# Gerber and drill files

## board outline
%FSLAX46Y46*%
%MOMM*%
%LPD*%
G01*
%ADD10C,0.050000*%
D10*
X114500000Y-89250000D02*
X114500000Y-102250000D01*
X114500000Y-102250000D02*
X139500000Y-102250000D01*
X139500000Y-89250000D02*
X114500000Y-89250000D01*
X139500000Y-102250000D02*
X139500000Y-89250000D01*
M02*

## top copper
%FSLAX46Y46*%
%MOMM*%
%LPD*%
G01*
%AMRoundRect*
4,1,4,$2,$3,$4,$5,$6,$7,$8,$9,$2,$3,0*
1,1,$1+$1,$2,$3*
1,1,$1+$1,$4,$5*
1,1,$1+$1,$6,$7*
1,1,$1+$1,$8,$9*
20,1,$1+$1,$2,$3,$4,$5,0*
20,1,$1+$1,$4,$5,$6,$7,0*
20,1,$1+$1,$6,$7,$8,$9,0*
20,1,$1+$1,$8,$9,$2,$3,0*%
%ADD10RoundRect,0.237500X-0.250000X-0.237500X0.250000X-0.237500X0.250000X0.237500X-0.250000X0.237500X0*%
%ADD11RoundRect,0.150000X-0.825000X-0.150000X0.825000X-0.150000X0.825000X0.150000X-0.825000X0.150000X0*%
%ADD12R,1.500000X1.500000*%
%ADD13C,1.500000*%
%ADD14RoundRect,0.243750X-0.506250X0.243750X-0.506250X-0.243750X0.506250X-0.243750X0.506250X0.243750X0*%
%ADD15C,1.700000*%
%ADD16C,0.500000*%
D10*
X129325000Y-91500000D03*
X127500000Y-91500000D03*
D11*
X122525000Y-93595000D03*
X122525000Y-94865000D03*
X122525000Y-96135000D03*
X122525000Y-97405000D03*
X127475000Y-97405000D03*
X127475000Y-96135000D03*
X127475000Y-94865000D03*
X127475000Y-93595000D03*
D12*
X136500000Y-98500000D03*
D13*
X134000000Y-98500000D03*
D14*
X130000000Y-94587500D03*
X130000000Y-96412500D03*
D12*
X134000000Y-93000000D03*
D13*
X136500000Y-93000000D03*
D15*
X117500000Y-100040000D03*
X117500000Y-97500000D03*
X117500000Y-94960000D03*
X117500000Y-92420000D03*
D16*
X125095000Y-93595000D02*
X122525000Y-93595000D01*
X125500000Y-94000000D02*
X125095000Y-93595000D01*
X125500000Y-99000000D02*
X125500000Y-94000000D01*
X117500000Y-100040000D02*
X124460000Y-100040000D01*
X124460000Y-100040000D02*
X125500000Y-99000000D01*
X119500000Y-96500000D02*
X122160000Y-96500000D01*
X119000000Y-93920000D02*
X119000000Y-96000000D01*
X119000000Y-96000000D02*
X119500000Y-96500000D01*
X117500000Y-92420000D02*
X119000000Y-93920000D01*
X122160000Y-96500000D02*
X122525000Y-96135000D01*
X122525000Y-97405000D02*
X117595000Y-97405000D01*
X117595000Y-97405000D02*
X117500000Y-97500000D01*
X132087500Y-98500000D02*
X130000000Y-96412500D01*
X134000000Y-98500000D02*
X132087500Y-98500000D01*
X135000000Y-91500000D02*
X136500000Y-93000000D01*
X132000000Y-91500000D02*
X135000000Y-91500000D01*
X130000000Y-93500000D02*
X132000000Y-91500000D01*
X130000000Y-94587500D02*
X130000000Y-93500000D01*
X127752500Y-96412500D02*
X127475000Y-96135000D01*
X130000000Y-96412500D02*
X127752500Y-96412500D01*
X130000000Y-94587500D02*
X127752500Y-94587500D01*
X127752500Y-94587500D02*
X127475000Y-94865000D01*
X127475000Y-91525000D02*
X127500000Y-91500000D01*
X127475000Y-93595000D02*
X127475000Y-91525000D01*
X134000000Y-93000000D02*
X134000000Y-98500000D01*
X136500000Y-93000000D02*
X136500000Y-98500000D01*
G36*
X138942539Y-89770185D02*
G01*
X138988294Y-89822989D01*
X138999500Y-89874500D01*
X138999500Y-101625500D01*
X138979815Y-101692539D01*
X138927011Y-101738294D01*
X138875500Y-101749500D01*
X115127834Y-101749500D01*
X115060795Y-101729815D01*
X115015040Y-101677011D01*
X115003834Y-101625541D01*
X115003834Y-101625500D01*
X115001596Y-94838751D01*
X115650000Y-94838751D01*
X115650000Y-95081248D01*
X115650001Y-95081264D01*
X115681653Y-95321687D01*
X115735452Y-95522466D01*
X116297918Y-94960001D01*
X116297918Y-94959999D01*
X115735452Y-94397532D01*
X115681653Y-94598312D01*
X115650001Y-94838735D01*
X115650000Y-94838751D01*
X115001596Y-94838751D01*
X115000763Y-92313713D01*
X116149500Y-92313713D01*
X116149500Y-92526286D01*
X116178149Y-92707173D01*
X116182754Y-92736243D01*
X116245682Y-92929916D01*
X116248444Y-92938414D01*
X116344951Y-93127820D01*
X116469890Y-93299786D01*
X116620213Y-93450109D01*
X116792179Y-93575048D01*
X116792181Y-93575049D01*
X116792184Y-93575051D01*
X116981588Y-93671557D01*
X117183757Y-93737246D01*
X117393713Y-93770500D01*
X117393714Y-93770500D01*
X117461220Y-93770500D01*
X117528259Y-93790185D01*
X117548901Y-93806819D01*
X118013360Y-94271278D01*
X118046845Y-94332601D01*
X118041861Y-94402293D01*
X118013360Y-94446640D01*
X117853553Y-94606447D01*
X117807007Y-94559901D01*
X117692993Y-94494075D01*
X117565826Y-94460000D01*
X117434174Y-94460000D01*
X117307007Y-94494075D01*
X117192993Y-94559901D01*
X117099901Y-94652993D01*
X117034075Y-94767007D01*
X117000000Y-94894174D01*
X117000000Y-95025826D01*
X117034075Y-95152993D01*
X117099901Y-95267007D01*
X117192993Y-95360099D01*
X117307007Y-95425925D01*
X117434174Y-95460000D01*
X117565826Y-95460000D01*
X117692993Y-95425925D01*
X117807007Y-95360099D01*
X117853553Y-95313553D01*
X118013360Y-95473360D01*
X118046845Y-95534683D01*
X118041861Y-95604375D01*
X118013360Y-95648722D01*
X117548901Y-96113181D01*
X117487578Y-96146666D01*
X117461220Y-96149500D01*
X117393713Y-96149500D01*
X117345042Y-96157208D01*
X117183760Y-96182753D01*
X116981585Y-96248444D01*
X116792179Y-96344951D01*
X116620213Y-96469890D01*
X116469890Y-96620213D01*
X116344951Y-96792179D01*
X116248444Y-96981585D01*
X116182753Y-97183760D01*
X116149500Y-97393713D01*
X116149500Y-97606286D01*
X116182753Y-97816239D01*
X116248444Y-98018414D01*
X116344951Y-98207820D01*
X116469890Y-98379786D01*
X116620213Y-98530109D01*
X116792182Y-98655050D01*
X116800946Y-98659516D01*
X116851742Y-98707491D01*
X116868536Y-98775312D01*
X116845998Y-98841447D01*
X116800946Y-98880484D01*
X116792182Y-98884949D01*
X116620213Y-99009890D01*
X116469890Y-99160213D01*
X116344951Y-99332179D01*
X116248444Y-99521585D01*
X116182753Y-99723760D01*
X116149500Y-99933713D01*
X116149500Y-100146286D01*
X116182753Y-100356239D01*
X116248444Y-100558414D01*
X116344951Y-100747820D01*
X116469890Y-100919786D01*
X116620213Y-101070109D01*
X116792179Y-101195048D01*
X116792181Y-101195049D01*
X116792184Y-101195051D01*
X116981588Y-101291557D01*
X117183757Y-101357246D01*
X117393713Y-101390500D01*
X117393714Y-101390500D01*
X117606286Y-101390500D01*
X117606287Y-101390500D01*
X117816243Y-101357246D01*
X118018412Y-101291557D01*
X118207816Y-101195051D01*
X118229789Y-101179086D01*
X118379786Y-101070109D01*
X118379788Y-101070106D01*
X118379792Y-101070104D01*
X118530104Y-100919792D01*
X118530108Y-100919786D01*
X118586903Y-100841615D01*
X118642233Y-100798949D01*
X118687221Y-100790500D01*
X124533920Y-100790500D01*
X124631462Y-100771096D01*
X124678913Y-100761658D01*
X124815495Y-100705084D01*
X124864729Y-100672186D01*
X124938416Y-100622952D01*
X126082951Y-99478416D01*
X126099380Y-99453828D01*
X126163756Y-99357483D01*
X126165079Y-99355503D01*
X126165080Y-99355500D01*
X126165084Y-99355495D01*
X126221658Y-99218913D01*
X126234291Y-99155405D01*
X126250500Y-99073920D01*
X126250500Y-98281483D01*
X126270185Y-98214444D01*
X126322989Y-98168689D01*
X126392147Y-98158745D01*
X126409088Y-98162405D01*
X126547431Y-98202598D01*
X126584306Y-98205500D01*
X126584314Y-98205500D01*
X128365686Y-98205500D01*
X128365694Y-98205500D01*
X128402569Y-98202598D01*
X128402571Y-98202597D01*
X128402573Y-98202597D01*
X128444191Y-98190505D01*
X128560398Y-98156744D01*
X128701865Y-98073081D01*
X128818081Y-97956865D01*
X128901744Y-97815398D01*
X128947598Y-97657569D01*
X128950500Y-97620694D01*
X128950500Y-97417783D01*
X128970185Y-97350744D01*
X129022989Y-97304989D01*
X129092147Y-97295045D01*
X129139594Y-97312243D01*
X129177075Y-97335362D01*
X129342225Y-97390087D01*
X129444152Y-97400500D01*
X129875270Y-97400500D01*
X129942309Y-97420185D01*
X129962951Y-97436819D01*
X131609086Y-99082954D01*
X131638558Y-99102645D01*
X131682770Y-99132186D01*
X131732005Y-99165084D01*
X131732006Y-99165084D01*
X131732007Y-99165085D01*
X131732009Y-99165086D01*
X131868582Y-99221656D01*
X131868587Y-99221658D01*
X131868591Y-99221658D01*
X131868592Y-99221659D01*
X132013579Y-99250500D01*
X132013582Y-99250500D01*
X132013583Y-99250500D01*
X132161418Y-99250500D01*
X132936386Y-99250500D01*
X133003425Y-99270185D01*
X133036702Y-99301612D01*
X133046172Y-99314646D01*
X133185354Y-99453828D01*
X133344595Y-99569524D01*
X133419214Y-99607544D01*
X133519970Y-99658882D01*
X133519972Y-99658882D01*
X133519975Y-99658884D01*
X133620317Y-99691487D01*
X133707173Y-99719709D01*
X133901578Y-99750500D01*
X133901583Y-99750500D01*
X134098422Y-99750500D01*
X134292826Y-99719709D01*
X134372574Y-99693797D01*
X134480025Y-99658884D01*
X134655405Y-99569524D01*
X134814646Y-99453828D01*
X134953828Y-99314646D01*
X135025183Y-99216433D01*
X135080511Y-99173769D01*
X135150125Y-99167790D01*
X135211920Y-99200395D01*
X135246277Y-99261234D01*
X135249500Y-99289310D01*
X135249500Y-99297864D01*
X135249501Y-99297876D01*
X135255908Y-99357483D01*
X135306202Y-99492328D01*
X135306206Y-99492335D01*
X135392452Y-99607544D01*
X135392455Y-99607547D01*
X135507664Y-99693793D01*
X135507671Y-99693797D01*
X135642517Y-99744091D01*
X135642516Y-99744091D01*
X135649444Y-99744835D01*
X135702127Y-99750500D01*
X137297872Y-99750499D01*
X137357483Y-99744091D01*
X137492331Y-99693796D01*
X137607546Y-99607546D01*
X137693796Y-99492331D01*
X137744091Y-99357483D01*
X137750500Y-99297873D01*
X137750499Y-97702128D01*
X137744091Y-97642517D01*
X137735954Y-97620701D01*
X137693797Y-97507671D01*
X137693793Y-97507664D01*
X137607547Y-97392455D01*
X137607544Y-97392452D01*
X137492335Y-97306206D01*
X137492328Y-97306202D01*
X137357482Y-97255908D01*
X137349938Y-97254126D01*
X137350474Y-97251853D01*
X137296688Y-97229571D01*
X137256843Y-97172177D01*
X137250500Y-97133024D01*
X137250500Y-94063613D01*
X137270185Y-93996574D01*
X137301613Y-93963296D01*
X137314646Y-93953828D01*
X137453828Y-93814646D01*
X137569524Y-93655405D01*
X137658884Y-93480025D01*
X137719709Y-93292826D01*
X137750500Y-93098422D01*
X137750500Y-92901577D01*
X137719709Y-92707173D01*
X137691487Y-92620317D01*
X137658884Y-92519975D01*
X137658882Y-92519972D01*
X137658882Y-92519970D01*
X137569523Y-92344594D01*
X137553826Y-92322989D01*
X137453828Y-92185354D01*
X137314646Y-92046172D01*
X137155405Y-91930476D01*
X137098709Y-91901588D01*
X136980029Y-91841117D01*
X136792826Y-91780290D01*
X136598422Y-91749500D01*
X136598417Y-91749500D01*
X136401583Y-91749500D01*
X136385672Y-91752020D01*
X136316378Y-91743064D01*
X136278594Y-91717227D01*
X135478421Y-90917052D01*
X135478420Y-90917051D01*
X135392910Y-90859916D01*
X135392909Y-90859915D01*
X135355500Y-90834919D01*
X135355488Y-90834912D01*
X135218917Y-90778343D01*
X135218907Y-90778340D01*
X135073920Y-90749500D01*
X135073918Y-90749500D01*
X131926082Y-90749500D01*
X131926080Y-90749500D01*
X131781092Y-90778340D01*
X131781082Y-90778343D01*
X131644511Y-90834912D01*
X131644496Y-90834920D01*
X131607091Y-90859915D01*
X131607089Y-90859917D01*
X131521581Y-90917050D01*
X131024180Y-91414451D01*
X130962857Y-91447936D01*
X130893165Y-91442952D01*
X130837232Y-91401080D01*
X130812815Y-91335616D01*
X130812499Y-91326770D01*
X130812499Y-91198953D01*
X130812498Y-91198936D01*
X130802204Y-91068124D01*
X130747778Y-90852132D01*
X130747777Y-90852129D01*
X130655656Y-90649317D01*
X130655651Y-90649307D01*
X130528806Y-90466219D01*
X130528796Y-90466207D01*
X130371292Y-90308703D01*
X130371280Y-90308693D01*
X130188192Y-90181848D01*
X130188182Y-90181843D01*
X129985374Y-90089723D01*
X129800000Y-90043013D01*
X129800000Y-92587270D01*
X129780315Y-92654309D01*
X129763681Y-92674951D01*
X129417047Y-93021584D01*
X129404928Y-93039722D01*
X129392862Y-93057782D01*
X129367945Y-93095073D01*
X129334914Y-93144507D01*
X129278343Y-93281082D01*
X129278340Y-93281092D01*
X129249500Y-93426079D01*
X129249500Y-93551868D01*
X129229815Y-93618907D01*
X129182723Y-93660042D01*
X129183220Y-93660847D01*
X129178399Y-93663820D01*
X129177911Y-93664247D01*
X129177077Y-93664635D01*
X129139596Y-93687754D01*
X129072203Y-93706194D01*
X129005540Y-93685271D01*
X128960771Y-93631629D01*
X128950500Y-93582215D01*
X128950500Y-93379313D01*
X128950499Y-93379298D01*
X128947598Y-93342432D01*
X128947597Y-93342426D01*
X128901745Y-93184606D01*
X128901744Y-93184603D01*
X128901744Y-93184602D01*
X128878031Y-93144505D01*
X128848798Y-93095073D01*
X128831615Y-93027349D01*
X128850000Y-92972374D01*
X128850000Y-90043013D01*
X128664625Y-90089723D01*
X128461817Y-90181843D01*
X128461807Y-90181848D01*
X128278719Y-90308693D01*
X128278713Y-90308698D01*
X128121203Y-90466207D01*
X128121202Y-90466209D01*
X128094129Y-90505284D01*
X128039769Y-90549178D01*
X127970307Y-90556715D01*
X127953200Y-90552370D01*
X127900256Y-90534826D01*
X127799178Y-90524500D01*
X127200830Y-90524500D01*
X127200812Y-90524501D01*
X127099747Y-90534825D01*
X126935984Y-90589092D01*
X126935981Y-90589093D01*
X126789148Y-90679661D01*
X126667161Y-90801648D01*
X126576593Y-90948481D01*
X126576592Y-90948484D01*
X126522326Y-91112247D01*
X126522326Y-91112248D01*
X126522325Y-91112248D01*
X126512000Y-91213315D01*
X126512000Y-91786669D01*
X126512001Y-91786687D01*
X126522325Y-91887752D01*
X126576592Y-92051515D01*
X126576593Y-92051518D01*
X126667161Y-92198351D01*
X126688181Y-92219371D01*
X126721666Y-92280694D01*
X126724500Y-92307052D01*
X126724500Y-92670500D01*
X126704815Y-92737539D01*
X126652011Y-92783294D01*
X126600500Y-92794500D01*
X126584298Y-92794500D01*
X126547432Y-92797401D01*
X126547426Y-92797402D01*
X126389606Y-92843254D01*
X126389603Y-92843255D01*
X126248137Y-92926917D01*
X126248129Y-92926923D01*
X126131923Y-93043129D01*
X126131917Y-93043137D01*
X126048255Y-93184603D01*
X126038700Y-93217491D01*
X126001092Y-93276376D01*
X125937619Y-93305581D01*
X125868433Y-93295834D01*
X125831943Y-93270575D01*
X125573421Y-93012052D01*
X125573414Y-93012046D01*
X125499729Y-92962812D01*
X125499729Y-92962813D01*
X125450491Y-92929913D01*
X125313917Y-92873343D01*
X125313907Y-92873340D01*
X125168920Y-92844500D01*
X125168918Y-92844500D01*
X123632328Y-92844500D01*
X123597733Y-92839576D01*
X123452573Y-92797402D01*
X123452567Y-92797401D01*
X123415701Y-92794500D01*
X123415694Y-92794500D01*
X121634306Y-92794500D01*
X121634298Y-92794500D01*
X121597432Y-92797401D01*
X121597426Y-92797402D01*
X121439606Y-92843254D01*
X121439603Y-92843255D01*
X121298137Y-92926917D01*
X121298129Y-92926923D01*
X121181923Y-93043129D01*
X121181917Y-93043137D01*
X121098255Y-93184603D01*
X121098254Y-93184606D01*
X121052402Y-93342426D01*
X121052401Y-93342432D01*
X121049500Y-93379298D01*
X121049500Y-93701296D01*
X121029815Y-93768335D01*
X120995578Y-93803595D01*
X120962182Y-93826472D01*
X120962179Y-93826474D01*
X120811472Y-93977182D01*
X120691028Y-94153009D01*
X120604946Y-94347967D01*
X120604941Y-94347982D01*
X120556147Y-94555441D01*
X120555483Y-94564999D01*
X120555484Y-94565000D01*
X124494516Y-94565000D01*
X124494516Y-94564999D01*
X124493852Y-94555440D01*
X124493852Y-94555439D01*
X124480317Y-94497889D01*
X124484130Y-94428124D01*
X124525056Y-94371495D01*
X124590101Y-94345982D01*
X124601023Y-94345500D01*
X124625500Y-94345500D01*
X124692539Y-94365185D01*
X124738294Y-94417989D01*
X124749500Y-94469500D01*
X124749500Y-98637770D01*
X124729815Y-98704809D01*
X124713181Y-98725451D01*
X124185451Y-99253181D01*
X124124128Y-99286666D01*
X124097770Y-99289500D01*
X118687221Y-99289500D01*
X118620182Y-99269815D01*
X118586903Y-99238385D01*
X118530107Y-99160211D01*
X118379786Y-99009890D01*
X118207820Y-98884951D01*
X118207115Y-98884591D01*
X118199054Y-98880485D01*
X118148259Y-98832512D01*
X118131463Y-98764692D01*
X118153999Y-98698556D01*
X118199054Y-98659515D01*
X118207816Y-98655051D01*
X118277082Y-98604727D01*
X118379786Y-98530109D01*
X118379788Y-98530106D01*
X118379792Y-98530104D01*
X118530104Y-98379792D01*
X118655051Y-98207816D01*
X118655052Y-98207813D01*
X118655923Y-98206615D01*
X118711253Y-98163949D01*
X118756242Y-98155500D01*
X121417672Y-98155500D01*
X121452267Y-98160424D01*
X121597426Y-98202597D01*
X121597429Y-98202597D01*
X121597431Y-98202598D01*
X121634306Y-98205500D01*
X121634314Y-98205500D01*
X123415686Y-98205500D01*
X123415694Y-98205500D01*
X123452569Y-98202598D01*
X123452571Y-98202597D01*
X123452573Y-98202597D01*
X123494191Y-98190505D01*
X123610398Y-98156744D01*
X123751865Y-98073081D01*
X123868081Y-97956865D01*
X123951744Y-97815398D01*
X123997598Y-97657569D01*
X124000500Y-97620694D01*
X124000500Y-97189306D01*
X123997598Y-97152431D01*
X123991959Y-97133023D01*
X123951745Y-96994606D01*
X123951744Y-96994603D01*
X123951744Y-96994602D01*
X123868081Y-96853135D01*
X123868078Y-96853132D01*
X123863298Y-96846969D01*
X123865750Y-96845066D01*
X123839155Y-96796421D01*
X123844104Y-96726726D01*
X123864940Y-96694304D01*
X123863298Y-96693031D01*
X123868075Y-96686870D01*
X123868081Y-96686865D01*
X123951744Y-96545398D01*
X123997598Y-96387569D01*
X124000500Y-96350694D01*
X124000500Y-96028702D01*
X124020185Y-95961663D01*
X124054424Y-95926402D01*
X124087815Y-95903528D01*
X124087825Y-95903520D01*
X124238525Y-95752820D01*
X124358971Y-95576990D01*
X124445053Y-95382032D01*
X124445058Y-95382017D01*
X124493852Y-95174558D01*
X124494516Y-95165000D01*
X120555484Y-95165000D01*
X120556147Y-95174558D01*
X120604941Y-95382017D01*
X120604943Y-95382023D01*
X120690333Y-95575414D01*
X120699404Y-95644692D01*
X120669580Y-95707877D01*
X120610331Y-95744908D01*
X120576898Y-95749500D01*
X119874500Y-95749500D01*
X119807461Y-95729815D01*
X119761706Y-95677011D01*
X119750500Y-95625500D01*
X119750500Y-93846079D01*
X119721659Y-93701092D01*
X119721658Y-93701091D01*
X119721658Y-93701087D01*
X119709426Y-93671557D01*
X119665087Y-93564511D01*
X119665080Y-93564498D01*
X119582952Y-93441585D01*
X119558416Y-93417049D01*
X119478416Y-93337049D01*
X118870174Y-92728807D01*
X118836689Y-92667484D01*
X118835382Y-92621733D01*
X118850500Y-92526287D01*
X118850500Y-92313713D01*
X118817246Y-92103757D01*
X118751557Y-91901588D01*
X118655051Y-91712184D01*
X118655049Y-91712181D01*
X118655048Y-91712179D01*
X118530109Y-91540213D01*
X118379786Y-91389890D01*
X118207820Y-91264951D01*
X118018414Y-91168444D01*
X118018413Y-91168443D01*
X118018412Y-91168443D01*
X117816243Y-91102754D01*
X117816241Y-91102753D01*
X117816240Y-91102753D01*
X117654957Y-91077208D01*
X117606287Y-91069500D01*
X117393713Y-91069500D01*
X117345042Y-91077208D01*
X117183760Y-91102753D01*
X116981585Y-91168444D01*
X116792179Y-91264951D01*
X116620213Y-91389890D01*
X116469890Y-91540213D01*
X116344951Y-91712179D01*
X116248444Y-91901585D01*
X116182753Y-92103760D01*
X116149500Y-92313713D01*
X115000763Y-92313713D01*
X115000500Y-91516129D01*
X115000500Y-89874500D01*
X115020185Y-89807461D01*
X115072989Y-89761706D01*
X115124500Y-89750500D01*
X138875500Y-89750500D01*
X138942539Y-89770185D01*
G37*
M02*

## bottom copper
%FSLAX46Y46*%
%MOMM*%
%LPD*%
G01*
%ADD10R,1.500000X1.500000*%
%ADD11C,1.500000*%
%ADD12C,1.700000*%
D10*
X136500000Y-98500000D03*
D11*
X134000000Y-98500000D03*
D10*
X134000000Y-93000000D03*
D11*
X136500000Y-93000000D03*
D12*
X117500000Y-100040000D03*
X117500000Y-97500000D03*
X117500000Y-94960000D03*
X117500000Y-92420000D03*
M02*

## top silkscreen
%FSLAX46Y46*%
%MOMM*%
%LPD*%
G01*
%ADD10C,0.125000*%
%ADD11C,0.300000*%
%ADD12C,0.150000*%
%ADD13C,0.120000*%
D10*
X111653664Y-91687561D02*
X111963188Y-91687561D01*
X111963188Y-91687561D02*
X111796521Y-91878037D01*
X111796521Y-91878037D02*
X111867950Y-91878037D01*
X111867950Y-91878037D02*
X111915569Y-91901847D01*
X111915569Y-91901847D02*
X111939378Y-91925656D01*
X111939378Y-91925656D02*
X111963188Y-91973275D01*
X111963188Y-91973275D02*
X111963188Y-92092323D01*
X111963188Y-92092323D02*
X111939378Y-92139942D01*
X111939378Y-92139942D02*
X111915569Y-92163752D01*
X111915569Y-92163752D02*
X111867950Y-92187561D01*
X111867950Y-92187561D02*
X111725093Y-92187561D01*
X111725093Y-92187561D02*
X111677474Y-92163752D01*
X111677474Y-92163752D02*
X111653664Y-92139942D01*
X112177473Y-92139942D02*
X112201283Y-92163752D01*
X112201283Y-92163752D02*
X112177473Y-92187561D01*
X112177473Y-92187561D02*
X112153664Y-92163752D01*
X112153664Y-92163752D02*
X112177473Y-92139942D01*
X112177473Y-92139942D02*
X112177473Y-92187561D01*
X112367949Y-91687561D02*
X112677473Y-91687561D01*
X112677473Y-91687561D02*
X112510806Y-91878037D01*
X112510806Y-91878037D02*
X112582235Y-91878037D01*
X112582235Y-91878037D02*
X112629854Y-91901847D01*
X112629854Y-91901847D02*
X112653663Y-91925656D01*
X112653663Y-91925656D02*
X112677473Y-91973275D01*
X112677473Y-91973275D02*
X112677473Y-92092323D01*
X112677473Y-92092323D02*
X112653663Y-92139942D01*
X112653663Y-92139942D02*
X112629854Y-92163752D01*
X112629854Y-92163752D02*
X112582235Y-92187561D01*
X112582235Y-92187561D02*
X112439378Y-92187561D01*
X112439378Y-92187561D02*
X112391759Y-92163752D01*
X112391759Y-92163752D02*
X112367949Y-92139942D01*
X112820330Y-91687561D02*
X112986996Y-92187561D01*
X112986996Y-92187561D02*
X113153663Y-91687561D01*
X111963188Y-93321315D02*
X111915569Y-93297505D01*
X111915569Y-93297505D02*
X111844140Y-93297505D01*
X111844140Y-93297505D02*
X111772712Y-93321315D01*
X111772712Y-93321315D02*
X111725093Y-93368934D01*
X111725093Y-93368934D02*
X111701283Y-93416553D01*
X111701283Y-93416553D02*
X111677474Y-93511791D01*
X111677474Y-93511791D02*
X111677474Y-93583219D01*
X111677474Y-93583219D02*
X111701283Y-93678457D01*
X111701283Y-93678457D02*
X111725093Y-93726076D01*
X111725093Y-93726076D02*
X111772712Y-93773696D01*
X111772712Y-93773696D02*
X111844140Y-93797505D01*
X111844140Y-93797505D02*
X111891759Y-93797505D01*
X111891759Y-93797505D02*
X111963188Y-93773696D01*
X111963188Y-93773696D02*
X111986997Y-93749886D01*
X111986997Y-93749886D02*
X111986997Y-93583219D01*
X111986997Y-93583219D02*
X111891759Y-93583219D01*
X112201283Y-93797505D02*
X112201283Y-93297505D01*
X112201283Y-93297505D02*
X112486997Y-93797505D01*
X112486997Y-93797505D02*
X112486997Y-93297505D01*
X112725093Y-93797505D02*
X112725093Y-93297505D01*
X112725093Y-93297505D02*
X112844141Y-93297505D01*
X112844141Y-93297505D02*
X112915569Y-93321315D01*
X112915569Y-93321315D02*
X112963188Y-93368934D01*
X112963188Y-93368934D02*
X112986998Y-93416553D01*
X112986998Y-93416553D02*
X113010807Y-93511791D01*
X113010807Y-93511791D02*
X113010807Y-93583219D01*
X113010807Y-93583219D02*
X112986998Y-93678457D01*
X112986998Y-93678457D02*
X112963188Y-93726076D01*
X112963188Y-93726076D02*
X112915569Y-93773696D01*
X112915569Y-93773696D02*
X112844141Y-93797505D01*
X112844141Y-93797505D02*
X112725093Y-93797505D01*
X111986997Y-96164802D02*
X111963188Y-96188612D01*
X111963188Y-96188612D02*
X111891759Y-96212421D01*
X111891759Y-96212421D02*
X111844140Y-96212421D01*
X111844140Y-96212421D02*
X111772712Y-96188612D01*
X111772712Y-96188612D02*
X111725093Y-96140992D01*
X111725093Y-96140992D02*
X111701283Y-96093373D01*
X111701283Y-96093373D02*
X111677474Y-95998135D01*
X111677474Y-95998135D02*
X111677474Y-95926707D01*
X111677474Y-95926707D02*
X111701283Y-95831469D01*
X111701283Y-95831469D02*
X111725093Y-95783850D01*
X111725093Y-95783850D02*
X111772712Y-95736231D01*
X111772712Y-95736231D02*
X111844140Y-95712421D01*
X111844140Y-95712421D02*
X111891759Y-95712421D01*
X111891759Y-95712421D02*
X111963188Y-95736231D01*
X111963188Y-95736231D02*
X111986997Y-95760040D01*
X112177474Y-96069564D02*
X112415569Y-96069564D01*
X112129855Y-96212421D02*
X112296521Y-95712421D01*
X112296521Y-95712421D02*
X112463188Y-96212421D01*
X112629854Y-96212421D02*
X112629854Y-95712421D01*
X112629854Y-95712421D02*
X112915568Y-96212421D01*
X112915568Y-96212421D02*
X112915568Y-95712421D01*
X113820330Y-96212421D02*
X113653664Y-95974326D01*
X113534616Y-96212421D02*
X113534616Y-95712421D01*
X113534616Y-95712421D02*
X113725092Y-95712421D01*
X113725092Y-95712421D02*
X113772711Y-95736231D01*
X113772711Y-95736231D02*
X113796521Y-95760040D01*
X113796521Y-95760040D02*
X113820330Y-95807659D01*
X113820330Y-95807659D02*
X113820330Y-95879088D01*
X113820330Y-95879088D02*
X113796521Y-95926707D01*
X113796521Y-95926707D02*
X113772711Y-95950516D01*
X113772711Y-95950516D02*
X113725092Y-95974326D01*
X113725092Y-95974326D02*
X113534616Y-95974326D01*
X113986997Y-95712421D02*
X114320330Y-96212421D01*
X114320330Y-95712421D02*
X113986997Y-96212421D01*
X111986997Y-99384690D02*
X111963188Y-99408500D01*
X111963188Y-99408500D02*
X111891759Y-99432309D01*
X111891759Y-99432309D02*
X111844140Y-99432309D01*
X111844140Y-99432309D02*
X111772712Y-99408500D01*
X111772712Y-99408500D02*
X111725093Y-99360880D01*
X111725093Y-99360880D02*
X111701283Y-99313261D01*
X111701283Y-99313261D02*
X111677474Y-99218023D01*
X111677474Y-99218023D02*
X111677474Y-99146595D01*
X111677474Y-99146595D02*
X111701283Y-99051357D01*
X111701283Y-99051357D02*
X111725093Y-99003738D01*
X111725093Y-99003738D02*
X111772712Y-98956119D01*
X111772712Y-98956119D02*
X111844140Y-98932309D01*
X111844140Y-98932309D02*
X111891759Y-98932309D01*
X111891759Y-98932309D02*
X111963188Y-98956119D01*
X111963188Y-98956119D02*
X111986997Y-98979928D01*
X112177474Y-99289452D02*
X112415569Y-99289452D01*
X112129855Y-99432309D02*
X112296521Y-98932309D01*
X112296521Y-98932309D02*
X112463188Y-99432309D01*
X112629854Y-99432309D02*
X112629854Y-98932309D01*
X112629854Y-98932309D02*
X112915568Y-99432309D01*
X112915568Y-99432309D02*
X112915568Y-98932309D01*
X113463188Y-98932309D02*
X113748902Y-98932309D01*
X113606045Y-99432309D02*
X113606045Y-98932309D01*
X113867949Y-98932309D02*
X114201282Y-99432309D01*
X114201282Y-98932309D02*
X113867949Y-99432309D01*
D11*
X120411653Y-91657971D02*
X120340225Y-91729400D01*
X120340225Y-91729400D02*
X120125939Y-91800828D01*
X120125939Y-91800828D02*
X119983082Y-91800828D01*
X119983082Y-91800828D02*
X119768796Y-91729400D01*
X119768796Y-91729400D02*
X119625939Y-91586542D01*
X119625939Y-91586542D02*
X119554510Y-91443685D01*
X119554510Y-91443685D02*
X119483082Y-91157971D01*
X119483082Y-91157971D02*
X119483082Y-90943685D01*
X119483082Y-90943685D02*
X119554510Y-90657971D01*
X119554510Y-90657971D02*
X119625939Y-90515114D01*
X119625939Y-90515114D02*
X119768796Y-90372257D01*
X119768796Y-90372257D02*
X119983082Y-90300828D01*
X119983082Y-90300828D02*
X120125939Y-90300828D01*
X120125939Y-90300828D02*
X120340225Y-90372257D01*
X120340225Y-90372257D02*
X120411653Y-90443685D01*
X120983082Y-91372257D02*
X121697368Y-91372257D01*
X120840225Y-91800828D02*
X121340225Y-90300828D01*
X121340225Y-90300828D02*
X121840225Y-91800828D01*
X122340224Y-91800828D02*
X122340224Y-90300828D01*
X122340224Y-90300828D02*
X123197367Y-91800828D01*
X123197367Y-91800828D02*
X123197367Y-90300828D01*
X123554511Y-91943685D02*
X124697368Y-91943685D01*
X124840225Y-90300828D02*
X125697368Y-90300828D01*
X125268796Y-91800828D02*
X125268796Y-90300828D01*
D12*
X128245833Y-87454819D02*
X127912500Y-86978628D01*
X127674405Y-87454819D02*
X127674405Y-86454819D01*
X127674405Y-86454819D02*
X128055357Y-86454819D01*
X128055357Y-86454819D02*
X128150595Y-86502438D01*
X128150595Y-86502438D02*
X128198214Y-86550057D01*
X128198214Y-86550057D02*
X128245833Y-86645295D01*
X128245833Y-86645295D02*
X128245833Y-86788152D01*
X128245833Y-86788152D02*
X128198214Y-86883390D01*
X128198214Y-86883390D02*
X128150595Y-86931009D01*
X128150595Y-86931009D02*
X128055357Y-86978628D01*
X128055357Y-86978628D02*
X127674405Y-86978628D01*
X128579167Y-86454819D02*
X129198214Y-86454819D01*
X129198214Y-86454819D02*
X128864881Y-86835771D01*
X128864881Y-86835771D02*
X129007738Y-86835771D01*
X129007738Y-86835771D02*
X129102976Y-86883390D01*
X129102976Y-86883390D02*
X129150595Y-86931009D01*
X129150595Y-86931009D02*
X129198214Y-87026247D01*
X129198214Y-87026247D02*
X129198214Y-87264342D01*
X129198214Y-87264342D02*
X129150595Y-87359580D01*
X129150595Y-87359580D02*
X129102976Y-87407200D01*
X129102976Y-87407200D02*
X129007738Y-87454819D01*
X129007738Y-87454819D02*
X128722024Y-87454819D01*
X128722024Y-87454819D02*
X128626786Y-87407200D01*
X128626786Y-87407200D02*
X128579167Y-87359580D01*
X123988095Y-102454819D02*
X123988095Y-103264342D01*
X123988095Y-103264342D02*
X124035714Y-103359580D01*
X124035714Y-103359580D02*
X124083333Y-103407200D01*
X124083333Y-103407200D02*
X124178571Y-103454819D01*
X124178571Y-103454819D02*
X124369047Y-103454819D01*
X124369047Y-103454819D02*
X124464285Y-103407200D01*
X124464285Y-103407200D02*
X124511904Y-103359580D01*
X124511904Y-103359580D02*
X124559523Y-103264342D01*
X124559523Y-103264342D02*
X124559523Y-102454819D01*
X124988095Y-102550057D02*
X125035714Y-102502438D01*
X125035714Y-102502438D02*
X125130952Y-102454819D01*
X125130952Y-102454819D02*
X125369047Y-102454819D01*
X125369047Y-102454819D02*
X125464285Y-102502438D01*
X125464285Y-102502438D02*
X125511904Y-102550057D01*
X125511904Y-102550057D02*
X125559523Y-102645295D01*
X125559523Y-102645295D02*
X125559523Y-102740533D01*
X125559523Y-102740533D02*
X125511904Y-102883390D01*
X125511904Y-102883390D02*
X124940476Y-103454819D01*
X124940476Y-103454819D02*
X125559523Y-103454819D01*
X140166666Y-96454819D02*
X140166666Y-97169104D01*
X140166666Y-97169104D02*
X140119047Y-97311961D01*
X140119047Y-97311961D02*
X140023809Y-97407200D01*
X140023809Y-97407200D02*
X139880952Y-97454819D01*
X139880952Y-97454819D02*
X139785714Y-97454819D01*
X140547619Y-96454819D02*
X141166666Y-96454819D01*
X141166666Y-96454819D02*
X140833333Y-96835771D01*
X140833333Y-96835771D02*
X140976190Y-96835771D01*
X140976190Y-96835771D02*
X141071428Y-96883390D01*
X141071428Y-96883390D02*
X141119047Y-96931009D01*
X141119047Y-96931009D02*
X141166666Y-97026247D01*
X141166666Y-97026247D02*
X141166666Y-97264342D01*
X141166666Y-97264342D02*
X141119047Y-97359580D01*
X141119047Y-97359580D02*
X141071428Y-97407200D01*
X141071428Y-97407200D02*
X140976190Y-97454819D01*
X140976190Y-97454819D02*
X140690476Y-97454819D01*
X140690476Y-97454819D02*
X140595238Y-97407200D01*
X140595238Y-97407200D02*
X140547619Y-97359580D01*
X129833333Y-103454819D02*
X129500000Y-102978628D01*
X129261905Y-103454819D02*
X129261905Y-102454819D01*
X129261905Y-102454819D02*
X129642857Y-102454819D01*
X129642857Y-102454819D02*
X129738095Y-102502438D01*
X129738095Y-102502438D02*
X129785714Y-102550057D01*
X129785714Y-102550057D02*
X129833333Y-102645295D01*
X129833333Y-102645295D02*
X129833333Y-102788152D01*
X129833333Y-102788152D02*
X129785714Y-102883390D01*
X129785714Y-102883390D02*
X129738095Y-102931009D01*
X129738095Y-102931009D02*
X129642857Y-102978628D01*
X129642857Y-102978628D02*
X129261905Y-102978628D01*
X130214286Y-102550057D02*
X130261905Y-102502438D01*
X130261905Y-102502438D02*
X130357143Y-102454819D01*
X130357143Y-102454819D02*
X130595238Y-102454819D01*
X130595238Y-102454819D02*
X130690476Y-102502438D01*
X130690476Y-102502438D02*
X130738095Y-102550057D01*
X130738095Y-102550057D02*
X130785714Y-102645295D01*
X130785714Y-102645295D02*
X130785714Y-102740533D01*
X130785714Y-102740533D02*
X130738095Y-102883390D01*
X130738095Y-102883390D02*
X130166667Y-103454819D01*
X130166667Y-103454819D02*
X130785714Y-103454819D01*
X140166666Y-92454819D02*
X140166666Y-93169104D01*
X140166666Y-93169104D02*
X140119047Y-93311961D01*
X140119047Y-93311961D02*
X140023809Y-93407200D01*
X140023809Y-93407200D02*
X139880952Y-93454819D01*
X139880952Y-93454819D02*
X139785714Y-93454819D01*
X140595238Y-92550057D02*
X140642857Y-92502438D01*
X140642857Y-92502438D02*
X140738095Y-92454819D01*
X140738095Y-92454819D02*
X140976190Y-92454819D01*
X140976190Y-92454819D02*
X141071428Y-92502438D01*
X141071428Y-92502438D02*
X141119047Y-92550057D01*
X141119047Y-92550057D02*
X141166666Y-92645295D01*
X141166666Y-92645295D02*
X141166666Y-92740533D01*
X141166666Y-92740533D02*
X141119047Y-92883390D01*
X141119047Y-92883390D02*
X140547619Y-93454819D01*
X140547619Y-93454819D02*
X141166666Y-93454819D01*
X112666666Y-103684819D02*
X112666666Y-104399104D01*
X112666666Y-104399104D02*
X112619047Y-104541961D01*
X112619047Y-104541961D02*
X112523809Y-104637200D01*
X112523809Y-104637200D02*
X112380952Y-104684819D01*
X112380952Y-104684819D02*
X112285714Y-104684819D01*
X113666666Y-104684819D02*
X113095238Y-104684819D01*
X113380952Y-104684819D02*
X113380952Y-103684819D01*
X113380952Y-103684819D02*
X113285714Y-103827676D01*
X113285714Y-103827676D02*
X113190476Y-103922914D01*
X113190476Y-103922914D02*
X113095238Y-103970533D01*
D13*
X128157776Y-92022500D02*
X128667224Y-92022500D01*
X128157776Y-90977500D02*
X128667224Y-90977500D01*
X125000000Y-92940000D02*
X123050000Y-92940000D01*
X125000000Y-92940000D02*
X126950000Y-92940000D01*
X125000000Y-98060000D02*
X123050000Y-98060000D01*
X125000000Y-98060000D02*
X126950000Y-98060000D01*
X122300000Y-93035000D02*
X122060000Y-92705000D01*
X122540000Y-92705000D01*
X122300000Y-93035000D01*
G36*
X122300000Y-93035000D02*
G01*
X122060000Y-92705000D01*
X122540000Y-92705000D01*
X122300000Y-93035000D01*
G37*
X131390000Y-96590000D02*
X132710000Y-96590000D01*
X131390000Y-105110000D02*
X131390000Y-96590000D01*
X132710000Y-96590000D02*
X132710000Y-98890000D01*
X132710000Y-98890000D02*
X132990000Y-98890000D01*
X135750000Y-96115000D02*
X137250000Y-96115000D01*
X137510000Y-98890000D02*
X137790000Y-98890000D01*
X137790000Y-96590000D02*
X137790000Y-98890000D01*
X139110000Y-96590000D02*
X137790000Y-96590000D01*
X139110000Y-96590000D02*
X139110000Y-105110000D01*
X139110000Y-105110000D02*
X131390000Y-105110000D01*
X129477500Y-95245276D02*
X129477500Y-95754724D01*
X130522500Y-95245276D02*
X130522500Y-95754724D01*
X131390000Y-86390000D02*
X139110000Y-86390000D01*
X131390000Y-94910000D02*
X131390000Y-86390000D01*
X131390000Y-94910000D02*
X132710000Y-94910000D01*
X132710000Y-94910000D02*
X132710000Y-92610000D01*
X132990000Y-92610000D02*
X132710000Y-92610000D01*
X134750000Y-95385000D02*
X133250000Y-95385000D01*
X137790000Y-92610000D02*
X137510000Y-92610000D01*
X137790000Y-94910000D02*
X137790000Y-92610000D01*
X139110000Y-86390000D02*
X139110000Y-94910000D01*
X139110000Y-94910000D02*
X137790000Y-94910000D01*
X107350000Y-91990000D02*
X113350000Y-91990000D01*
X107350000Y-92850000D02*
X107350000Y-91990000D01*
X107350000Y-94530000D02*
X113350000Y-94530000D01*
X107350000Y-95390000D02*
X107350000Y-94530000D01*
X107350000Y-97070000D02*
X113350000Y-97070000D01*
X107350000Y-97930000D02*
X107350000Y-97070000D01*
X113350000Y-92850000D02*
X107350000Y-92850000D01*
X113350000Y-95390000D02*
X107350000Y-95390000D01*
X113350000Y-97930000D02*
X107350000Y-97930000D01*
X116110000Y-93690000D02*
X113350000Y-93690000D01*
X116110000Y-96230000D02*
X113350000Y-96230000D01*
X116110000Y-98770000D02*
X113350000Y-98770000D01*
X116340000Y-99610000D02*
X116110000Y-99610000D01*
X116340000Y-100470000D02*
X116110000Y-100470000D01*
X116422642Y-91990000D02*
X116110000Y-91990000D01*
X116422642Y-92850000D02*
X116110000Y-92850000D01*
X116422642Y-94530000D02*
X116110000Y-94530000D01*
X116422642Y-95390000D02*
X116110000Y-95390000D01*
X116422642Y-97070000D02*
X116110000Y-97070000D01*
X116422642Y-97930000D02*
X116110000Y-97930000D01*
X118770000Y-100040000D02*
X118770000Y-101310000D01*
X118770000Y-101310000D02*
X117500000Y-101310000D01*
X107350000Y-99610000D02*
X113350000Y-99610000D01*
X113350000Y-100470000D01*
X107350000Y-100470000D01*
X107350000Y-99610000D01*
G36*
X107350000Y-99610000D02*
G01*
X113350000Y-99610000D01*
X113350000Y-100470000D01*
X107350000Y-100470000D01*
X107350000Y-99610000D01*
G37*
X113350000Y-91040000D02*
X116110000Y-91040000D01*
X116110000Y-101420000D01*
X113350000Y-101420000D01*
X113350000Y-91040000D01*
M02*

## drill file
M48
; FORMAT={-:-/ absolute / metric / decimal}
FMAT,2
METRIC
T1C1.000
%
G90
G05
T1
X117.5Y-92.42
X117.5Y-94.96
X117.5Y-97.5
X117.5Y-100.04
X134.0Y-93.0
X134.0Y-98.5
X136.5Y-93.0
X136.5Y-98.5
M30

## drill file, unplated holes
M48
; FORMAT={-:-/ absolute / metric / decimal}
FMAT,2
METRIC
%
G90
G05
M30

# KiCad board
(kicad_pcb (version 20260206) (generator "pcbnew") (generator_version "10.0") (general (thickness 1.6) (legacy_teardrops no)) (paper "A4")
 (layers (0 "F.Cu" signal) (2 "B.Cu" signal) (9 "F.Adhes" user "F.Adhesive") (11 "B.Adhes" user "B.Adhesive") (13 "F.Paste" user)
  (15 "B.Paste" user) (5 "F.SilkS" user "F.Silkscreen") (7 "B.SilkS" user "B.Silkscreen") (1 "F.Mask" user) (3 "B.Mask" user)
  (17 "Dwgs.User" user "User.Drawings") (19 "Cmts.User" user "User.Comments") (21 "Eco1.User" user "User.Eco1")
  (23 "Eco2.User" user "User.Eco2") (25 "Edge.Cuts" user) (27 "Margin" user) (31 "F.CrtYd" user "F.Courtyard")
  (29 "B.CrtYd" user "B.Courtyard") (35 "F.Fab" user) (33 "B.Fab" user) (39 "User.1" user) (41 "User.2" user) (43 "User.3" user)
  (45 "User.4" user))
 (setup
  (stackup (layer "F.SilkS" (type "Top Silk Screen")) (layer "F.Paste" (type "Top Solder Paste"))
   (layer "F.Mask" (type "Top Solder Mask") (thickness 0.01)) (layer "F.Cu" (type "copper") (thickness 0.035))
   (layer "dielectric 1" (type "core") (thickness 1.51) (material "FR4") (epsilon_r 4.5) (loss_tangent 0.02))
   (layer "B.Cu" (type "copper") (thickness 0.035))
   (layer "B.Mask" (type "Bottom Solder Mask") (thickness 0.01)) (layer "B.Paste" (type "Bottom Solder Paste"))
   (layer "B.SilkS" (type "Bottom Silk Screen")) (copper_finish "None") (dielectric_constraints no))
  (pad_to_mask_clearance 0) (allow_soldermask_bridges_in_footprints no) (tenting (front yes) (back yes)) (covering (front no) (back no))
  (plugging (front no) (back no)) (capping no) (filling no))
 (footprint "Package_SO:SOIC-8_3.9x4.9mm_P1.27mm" (layer "F.Cu") (at 125 95.5)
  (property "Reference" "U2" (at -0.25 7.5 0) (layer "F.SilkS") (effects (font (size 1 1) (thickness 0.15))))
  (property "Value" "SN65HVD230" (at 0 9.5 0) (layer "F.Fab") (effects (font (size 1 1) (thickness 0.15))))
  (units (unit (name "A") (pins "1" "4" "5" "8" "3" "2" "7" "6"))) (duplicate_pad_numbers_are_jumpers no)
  (fp_line (start 0 -2.56) (end -1.95 -2.56) (stroke (width 0.12) (type solid)) (layer "F.SilkS"))
  (fp_line (start 0 -2.56) (end 1.95 -2.56) (stroke (width 0.12) (type solid)) (layer "F.SilkS"))
  (fp_line (start 0 2.56) (end -1.95 2.56) (stroke (width 0.12) (type solid)) (layer "F.SilkS"))
  (fp_line (start 0 2.56) (end 1.95 2.56) (stroke (width 0.12) (type solid)) (layer "F.SilkS"))
  (fp_poly (pts (xy -2.7 -2.465) (xy -2.94 -2.795) (xy -2.46 -2.795)) (stroke (width 0.12) (type solid)) (fill yes) (layer "F.SilkS"))
  (pad "1" smd roundrect (at -2.475 -1.905) (size 1.95 0.6) (layers "F.Cu" "F.Mask" "F.Paste") (roundrect_rratio 0.25)
   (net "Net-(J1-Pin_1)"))
  (pad "2" smd roundrect (at -2.475 -0.635) (size 1.95 0.6) (layers "F.Cu" "F.Mask" "F.Paste") (roundrect_rratio 0.25) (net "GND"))
  (pad "3" smd roundrect (at -2.475 0.635) (size 1.95 0.6) (layers "F.Cu" "F.Mask" "F.Paste") (roundrect_rratio 0.25) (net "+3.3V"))
  (pad "4" smd roundrect (at -2.475 1.905) (size 1.95 0.6) (layers "F.Cu" "F.Mask" "F.Paste") (roundrect_rratio 0.25) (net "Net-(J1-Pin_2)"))
  (pad "5" smd roundrect (at 2.475 1.905) (size 1.95 0.6) (layers "F.Cu" "F.Mask" "F.Paste") (roundrect_rratio 0.25)
   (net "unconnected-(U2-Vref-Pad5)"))
  (pad "6" smd roundrect (at 2.475 0.635) (size 1.95 0.6) (layers "F.Cu" "F.Mask" "F.Paste") (roundrect_rratio 0.25) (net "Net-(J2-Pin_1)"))
  (pad "7" smd roundrect (at 2.475 -0.635) (size 1.95 0.6) (layers "F.Cu" "F.Mask" "F.Paste") (roundrect_rratio 0.25) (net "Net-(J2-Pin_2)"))
  (pad "8" smd roundrect (at 2.475 -1.905) (size 1.95 0.6) (layers "F.Cu" "F.Mask" "F.Paste") (roundrect_rratio 0.25) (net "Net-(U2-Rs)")))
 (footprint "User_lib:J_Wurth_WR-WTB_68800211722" (layer "F.Cu") (at 136.5 98.5 180)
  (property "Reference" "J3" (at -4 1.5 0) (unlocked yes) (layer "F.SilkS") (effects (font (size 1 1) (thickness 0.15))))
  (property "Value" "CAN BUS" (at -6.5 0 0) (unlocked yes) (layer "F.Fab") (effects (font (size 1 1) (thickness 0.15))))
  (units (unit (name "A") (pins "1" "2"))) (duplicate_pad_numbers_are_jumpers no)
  (fp_line (start 5.11 1.91) (end 3.79 1.91) (stroke (width 0.12) (type solid)) (layer "F.SilkS"))
  (fp_line (start 5.11 -6.61) (end 5.11 1.91) (stroke (width 0.12) (type default)) (layer "F.SilkS"))
  (fp_line (start 3.79 1.91) (end 3.79 -0.39) (stroke (width 0.12) (type solid)) (layer "F.SilkS"))
  (fp_line (start 3.79 -0.39) (end 3.51 -0.39) (stroke (width 0.12) (type solid)) (layer "F.SilkS"))
  (fp_line (start 0.75 2.385) (end -0.75 2.385) (stroke (width 0.12) (type solid)) (layer "F.SilkS"))
  (fp_line (start -1.01 -0.39) (end -1.29 -0.39) (stroke (width 0.12) (type solid)) (layer "F.SilkS"))
  (fp_line (start -1.29 1.91) (end -1.29 -0.39) (stroke (width 0.12) (type solid)) (layer "F.SilkS"))
  (fp_line (start -2.61 1.91) (end -1.29 1.91) (stroke (width 0.12) (type solid)) (layer "F.SilkS"))
  (fp_line (start -2.61 1.91) (end -2.61 -6.61) (stroke (width 0.12) (type default)) (layer "F.SilkS"))
  (fp_line (start -2.61 -6.61) (end 5.11 -6.61) (stroke (width 0.12) (type default)) (layer "F.SilkS"))
  (pad "1" thru_hole rect (at 0 0) (size 1.5 1.5) (drill 1) (layers "*.Cu" "*.Mask") (remove_unused_layers no) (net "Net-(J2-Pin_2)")
   (thermal_bridge_angle 45))
  (pad "2" thru_hole circle (at 2.5 0) (size 1.5 1.5) (drill 1) (layers "*.Cu" "*.Mask") (remove_unused_layers no) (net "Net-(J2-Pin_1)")))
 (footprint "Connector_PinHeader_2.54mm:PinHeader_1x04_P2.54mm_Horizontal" (layer "F.Cu") (at 117.5 100.04 180)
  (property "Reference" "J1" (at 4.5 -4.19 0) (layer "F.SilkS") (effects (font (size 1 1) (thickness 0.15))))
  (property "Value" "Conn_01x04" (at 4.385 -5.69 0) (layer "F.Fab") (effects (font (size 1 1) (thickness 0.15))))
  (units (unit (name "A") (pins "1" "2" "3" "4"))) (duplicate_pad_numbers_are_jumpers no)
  (fp_line (start 10.15 8.05) (end 4.15 8.05) (stroke (width 0.12) (type solid)) (layer "F.SilkS"))
  (fp_line (start 10.15 7.19) (end 10.15 8.05) (stroke (width 0.12) (type solid)) (layer "F.SilkS"))
  (fp_line (start 10.15 5.51) (end 4.15 5.51) (stroke (width 0.12) (type solid)) (layer "F.SilkS"))
  (fp_line (start 10.15 4.65) (end 10.15 5.51) (stroke (width 0.12) (type solid)) (layer "F.SilkS"))
  (fp_line (start 10.15 2.97) (end 4.15 2.97) (stroke (width 0.12) (type solid)) (layer "F.SilkS"))
  (fp_line (start 10.15 2.11) (end 10.15 2.97) (stroke (width 0.12) (type solid)) (layer "F.SilkS"))
  (fp_line (start 4.15 7.19) (end 10.15 7.19) (stroke (width 0.12) (type solid)) (layer "F.SilkS"))
  (fp_line (start 4.15 4.65) (end 10.15 4.65) (stroke (width 0.12) (type solid)) (layer "F.SilkS"))
  (fp_line (start 4.15 2.11) (end 10.15 2.11) (stroke (width 0.12) (type solid)) (layer "F.SilkS"))
  (fp_line (start 1.39 6.35) (end 4.15 6.35) (stroke (width 0.12) (type solid)) (layer "F.SilkS"))
  (fp_line (start 1.39 3.81) (end 4.15 3.81) (stroke (width 0.12) (type solid)) (layer "F.SilkS"))
  (fp_line (start 1.39 1.27) (end 4.15 1.27) (stroke (width 0.12) (type solid)) (layer "F.SilkS"))
  (fp_line (start 1.16 0.43) (end 1.39 0.43) (stroke (width 0.12) (type solid)) (layer "F.SilkS"))
  (fp_line (start 1.16 -0.43) (end 1.39 -0.43) (stroke (width 0.12) (type solid)) (layer "F.SilkS"))
  (fp_line (start 1.077358 8.05) (end 1.39 8.05) (stroke (width 0.12) (type solid)) (layer "F.SilkS"))
  (fp_line (start 1.077358 7.19) (end 1.39 7.19) (stroke (width 0.12) (type solid)) (layer "F.SilkS"))
  (fp_line (start 1.077358 5.51) (end 1.39 5.51) (stroke (width 0.12) (type solid)) (layer "F.SilkS"))
  (fp_line (start 1.077358 4.65) (end 1.39 4.65) (stroke (width 0.12) (type solid)) (layer "F.SilkS"))
  (fp_line (start 1.077358 2.97) (end 1.39 2.97) (stroke (width 0.12) (type solid)) (layer "F.SilkS"))
  (fp_line (start 1.077358 2.11) (end 1.39 2.11) (stroke (width 0.12) (type solid)) (layer "F.SilkS"))
  (fp_line (start -1.27 0) (end -1.27 -1.27) (stroke (width 0.12) (type solid)) (layer "F.SilkS"))
  (fp_line (start -1.27 -1.27) (end 0 -1.27) (stroke (width 0.12) (type solid)) (layer "F.SilkS"))
  (fp_rect (start 4.15 -0.43) (end 10.15 0.43) (stroke (width 0.12) (type solid)) (fill yes) (layer "F.SilkS"))
  (fp_rect (start 1.39 -1.38) (end 4.15 9) (stroke (width 0.12) (type solid)) (fill no) (layer "F.SilkS"))
  (pad "1" thru_hole circle (at 0 0 180) (size 1.7 1.7) (drill 1) (layers "*.Cu" "*.Mask") (remove_unused_layers no) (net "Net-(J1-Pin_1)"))
  (pad "2" thru_hole circle (at 0 2.54 180) (size 1.7 1.7) (drill 1) (layers "*.Cu" "*.Mask") (remove_unused_layers no)
   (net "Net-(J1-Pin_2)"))
  (pad "3" thru_hole circle (at 0 5.08 180) (size 1.7 1.7) (drill 1) (layers "*.Cu" "*.Mask") (remove_unused_layers no) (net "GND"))
  (pad "4" thru_hole circle (at 0 7.62 180) (size 1.7 1.7) (drill 1) (layers "*.Cu" "*.Mask") (remove_unused_layers no) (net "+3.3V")))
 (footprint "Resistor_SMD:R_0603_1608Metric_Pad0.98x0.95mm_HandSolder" (layer "F.Cu") (at 130 95.5 -90)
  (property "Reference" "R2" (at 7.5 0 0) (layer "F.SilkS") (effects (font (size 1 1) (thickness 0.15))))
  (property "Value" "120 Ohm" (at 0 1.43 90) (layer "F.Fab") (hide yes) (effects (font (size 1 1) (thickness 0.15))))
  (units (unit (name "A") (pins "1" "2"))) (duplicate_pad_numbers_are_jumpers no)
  (fp_line (start -0.254724 0.5225) (end 0.254724 0.5225) (stroke (width 0.12) (type solid)) (layer "F.SilkS"))
  (fp_line (start -0.254724 -0.5225) (end 0.254724 -0.5225) (stroke (width 0.12) (type solid)) (layer "F.SilkS"))
  (pad "1" smd roundrect (at -0.9125 0 270) (size 0.975 1.5) (layers "F.Cu" "F.Mask" "F.Paste") (roundrect_rratio 0.25)
   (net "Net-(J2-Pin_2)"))
  (pad "2" smd roundrect (at 0.9125 0 270) (size 0.975 1.5) (layers "F.Cu" "F.Mask" "F.Paste") (roundrect_rratio 0.25)
   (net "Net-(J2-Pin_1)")))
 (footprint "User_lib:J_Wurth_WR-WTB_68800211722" (layer "F.Cu") (at 134 93)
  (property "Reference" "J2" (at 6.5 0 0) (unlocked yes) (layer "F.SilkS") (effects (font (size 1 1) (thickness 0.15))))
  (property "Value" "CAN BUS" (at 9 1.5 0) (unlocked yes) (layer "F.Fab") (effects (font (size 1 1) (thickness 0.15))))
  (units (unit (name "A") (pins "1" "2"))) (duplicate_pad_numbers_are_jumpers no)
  (fp_line (start -2.61 -6.61) (end 5.11 -6.61) (stroke (width 0.12) (type default)) (layer "F.SilkS"))
  (fp_line (start -2.61 1.91) (end -2.61 -6.61) (stroke (width 0.12) (type default)) (layer "F.SilkS"))
  (fp_line (start -2.61 1.91) (end -1.29 1.91) (stroke (width 0.12) (type solid)) (layer "F.SilkS"))
  (fp_line (start -1.29 1.91) (end -1.29 -0.39) (stroke (width 0.12) (type solid)) (layer "F.SilkS"))
  (fp_line (start -1.01 -0.39) (end -1.29 -0.39) (stroke (width 0.12) (type solid)) (layer "F.SilkS"))
  (fp_line (start 0.75 2.385) (end -0.75 2.385) (stroke (width 0.12) (type solid)) (layer "F.SilkS"))
  (fp_line (start 3.79 -0.39) (end 3.51 -0.39) (stroke (width 0.12) (type solid)) (layer "F.SilkS"))
  (fp_line (start 3.79 1.91) (end 3.79 -0.39) (stroke (width 0.12) (type solid)) (layer "F.SilkS"))
  (fp_line (start 5.11 -6.61) (end 5.11 1.91) (stroke (width 0.12) (type default)) (layer "F.SilkS"))
  (fp_line (start 5.11 1.91) (end 3.79 1.91) (stroke (width 0.12) (type solid)) (layer "F.SilkS"))
  (pad "1" thru_hole rect (at 0 0 180) (size 1.5 1.5) (drill 1) (layers "*.Cu" "*.Mask") (remove_unused_layers no) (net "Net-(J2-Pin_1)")
   (thermal_bridge_angle 45))
  (pad "2" thru_hole circle (at 2.5 0 180) (size 1.5 1.5) (drill 1) (layers "*.Cu" "*.Mask") (remove_unused_layers no)
   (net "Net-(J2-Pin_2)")))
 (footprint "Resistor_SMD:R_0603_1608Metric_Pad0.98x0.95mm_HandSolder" (layer "F.Cu") (at 128.4125 91.5)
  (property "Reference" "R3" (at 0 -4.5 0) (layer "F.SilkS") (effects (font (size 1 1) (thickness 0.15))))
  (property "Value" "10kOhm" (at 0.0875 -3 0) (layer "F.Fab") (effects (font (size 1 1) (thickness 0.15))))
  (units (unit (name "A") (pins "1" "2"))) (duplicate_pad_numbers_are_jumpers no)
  (fp_line (start -0.254724 -0.5225) (end 0.254724 -0.5225) (stroke (width 0.12) (type solid)) (layer "F.SilkS"))
  (fp_line (start -0.254724 0.5225) (end 0.254724 0.5225) (stroke (width 0.12) (type solid)) (layer "F.SilkS"))
  (pad "1" smd roundrect (at -0.9125 0) (size 0.975 0.95) (layers "F.Cu" "F.Mask" "F.Paste") (roundrect_rratio 0.25) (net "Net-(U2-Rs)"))
  (pad "2" smd roundrect (at 0.9125 0) (size 0.975 0.95) (layers "F.Cu" "F.Mask" "F.Paste") (roundrect_rratio 0.25) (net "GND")))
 (gr_line (start 114.5 89.25) (end 114.5 102.25) (stroke (width 0.05) (type default)) (layer "Edge.Cuts"))
 (gr_line (start 114.5 102.25) (end 139.5 102.25) (stroke (width 0.05) (type default)) (layer "Edge.Cuts"))
 (gr_line (start 139.5 89.25) (end 114.5 89.25) (stroke (width 0.05) (type default)) (layer "Edge.Cuts"))
 (gr_line (start 139.5 102.25) (end 139.5 89.25) (stroke (width 0.05) (type default)) (layer "Edge.Cuts"))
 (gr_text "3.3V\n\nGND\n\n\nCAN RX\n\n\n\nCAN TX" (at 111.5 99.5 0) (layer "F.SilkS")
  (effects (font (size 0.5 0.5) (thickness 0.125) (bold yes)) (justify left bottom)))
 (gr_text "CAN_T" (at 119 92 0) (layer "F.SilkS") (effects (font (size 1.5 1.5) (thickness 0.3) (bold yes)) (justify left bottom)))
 (segment (start 125.5 94) (end 125.095 93.595) (width 0.5) (layer "F.Cu") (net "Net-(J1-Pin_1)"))
 (segment (start 117.5 100.04) (end 124.46 100.04) (width 0.5) (layer "F.Cu") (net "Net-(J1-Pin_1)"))
 (segment (start 124.46 100.04) (end 125.5 99) (width 0.5) (layer "F.Cu") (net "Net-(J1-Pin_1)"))
 (segment (start 125.5 99) (end 125.5 94) (width 0.5) (layer "F.Cu") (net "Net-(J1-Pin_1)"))
 (segment (start 125.095 93.595) (end 122.525 93.595) (width 0.5) (layer "F.Cu") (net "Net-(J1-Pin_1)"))
 (segment (start 119 96) (end 119.5 96.5) (width 0.5) (layer "F.Cu") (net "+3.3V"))
 (segment (start 119.5 96.5) (end 122.16 96.5) (width 0.5) (layer "F.Cu") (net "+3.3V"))
 (segment (start 117.5 92.42) (end 119 93.92) (width 0.5) (layer "F.Cu") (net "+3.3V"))
 (segment (start 122.16 96.5) (end 122.525 96.135) (width 0.5) (layer "F.Cu") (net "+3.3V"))
 (segment (start 119 93.92) (end 119 96) (width 0.5) (layer "F.Cu") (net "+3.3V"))
 (segment (start 117.595 97.405) (end 117.5 97.5) (width 0.5) (layer "F.Cu") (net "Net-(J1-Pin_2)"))
 (segment (start 122.525 97.405) (end 117.595 97.405) (width 0.5) (layer "F.Cu") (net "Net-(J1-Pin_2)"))
 (segment (start 130 96.4125) (end 127.7525 96.4125) (width 0.5) (layer "F.Cu") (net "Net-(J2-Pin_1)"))
 (segment (start 134 93) (end 134 98.5) (width 0.5) (layer "F.Cu") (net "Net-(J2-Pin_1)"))
 (segment (start 132.0875 98.5) (end 130 96.4125) (width 0.5) (layer "F.Cu") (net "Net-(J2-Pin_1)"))
 (segment (start 127.7525 96.4125) (end 127.475 96.135) (width 0.5) (layer "F.Cu") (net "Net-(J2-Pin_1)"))
 (segment (start 134 98.5) (end 132.0875 98.5) (width 0.5) (layer "F.Cu") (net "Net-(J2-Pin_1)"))
 (segment (start 130 93.5) (end 132 91.5) (width 0.5) (layer "F.Cu") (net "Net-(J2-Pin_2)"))
 (segment (start 135 91.5) (end 136.5 93) (width 0.5) (layer "F.Cu") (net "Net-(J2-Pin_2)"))
 (segment (start 130 94.5875) (end 130 93.5) (width 0.5) (layer "F.Cu") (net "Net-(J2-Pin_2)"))
 (segment (start 127.7525 94.5875) (end 127.475 94.865) (width 0.5) (layer "F.Cu") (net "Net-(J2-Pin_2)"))
 (segment (start 136.5 93) (end 136.5 98.5) (width 0.5) (layer "F.Cu") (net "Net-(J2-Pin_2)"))
 (segment (start 130 94.5875) (end 127.7525 94.5875) (width 0.5) (layer "F.Cu") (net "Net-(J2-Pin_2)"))
 (segment (start 132 91.5) (end 135 91.5) (width 0.5) (layer "F.Cu") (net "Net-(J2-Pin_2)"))
 (segment (start 127.475 93.595) (end 127.475 91.525) (width 0.5) (layer "F.Cu") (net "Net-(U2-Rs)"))
 (segment (start 127.475 91.525) (end 127.5 91.5) (width 0.5) (layer "F.Cu") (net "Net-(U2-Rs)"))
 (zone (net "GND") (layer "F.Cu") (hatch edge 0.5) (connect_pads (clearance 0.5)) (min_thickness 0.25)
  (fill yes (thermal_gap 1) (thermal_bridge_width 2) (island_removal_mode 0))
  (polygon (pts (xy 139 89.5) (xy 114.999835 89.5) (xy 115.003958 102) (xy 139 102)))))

